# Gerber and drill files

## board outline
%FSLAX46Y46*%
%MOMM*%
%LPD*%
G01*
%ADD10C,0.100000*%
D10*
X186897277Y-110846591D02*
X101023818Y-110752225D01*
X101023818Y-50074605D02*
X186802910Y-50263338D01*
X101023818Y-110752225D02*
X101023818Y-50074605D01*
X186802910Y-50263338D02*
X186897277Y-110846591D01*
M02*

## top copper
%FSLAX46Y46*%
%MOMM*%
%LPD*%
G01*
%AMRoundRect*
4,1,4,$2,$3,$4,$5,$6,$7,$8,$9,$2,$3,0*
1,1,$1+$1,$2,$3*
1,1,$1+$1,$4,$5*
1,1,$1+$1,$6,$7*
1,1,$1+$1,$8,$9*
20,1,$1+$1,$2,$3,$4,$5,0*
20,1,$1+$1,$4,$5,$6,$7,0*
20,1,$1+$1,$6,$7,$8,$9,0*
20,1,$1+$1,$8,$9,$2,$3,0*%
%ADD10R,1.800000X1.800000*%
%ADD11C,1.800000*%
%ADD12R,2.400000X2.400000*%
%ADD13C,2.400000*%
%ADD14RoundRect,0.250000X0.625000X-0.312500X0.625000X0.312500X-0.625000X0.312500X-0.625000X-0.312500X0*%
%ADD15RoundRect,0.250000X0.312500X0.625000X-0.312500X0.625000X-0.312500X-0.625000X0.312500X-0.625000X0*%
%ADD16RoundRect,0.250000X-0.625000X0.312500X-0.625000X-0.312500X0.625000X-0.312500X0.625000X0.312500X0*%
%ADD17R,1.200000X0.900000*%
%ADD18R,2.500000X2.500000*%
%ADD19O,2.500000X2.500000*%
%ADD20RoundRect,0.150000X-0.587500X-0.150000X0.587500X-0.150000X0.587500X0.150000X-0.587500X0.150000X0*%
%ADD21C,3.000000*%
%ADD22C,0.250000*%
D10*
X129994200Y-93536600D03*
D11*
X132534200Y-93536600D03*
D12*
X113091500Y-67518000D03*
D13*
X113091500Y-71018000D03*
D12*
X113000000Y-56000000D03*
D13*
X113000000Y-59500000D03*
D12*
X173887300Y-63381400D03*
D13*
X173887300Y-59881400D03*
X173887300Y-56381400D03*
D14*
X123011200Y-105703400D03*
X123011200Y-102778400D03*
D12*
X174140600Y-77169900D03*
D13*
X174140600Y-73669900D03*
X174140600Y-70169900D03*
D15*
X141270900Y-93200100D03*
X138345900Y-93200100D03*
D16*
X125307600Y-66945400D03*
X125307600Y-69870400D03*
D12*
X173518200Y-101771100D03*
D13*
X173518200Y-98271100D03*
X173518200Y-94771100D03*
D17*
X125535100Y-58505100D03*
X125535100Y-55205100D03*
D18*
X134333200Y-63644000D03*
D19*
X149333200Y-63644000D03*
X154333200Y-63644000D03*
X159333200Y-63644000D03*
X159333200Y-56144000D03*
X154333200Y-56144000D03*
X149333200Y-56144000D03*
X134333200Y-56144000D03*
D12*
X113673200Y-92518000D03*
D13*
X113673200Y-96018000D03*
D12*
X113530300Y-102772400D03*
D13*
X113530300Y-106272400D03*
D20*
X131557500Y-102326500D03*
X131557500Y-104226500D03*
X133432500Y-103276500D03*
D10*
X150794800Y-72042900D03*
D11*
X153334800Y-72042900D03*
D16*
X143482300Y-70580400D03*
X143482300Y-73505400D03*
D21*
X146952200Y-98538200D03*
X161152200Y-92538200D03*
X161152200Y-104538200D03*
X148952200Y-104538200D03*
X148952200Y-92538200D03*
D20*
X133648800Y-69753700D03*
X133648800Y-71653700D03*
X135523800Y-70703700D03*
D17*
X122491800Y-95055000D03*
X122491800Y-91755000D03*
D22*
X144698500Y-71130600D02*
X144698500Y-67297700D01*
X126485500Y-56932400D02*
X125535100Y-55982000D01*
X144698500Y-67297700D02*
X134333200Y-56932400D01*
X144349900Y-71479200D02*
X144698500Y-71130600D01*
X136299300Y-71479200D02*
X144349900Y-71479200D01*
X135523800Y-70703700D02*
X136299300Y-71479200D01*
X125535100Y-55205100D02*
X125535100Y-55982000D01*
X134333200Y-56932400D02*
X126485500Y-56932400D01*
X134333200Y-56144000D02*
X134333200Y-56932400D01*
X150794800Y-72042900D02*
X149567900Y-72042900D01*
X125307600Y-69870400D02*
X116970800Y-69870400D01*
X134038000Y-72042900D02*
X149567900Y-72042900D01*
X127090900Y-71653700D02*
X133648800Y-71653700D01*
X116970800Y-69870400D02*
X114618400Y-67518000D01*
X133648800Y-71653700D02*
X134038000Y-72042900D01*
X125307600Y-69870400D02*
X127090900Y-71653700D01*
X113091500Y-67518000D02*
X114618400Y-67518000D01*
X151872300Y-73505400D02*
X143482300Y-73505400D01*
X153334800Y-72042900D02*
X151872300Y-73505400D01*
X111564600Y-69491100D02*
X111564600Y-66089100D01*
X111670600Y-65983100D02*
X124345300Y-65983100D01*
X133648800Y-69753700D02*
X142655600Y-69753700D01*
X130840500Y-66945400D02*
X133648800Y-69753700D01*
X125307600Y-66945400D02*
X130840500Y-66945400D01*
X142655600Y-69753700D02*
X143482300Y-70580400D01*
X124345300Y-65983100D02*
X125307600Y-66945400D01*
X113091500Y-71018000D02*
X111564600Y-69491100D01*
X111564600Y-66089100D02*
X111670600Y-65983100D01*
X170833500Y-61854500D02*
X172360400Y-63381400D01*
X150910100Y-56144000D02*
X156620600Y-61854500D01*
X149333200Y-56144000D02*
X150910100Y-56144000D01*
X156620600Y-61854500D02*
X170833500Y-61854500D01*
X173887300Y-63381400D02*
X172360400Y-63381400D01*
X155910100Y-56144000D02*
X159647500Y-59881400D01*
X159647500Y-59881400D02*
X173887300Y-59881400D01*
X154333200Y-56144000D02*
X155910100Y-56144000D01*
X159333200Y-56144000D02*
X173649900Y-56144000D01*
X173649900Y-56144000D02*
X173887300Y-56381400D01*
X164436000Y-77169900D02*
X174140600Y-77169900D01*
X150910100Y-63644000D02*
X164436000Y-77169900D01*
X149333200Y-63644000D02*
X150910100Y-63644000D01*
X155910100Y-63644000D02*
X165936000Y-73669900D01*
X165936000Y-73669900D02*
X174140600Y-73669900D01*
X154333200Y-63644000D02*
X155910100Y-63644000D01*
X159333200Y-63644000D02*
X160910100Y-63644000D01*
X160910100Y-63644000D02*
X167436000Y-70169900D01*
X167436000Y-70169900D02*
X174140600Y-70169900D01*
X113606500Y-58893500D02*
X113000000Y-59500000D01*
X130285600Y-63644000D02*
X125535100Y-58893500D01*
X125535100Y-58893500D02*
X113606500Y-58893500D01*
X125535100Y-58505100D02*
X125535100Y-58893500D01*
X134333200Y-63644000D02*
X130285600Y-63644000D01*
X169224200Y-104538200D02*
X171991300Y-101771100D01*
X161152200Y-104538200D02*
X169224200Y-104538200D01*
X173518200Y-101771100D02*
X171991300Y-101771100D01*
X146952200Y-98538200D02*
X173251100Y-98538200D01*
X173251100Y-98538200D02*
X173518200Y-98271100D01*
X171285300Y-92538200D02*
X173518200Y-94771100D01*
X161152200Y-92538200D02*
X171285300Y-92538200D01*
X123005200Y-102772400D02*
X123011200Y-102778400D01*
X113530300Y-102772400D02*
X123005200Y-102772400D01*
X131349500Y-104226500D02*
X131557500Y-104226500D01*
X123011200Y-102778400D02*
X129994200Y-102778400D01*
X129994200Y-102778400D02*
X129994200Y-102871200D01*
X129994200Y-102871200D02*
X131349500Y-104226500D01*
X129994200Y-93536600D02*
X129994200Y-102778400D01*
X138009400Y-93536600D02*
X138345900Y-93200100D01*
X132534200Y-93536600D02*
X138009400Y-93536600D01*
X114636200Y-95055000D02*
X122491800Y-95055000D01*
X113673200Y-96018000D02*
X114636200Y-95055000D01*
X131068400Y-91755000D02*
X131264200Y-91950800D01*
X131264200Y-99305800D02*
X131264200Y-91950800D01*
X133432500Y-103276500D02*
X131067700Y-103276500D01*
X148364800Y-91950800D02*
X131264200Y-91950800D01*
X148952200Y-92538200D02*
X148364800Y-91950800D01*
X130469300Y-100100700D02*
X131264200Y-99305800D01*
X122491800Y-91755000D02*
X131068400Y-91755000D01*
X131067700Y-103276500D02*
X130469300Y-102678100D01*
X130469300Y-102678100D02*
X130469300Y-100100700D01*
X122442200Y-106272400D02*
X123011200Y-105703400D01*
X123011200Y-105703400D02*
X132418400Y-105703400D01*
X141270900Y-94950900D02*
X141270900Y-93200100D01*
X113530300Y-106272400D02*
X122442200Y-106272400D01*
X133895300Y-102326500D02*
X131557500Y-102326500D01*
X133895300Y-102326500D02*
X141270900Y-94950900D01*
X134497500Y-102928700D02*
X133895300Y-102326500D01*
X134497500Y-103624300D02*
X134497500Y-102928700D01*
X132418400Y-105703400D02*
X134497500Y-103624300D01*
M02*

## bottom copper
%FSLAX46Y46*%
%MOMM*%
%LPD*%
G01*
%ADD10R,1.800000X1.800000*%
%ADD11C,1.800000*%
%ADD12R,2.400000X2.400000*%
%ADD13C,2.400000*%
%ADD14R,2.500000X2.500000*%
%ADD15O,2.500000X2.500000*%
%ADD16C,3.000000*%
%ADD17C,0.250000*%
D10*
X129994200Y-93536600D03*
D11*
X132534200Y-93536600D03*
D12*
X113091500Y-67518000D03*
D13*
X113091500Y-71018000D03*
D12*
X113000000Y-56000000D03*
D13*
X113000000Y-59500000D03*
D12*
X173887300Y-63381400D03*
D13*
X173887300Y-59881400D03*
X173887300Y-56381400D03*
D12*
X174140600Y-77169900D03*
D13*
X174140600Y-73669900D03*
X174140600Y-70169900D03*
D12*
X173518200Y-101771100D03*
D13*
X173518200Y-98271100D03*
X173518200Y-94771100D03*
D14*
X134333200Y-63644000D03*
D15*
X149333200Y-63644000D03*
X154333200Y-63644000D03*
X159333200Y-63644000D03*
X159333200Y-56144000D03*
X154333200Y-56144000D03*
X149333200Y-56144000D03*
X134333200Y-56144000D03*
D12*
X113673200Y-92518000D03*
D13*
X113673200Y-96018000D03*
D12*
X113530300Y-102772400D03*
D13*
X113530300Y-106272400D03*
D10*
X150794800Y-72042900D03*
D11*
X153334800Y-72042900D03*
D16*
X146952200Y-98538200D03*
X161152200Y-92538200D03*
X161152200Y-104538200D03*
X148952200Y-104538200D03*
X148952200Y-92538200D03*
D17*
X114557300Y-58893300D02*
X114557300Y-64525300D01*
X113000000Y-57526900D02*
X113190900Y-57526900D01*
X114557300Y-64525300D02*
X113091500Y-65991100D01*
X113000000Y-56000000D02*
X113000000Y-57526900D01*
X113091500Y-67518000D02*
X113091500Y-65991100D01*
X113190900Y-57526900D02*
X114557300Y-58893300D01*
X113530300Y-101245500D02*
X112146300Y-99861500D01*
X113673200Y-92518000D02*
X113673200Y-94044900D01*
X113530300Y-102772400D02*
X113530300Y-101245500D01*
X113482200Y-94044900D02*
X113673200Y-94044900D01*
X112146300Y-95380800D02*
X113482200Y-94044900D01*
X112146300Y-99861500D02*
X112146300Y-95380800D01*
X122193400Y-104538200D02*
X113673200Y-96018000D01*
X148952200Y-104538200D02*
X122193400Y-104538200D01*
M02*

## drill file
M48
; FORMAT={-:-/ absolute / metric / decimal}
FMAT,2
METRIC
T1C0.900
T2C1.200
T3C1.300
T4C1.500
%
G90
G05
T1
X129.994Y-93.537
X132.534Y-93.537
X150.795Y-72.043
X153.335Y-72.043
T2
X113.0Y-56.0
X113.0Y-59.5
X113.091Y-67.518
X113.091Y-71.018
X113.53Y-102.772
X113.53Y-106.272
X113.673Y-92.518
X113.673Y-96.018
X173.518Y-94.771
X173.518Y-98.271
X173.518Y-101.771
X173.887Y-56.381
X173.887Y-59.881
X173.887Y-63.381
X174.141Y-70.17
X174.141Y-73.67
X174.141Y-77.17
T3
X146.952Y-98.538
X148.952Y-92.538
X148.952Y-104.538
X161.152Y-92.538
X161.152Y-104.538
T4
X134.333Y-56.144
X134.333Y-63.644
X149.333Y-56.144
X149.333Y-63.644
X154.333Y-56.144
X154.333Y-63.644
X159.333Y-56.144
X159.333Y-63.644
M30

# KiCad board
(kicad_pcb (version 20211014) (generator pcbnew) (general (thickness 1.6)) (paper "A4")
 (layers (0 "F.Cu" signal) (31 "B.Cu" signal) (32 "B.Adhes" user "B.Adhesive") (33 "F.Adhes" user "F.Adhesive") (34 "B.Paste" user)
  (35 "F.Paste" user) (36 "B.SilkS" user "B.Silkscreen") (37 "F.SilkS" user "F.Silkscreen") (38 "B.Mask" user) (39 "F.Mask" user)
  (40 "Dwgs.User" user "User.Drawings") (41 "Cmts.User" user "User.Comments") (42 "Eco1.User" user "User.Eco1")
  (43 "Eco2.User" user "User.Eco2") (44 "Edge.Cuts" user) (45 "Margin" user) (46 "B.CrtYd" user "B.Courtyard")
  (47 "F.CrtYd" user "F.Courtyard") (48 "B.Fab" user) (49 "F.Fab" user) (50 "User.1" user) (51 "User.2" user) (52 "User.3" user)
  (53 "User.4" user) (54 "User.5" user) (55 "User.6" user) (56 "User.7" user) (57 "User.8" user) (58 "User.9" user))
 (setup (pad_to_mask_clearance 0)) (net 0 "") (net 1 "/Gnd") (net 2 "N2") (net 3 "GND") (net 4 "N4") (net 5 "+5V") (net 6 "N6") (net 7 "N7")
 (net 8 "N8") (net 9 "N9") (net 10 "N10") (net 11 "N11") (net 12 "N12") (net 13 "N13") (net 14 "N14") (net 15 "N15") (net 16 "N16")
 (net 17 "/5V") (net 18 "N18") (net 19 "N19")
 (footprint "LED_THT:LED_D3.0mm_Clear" (layer "F.Cu") (at 129.9942 93.5366)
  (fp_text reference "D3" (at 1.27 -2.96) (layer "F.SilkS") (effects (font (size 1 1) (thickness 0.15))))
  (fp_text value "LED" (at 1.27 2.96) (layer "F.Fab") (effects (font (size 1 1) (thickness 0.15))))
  (pad "1" thru_hole rect (at 0 0) (size 1.8 1.8) (drill 0.9) (layers *.Cu *.Mask) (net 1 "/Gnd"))
  (pad "2" thru_hole circle (at 2.54 0) (size 1.8 1.8) (drill 0.9) (layers *.Cu *.Mask) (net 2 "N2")))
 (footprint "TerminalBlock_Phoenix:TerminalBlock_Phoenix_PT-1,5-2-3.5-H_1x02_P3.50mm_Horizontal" (layer "F.Cu") (at 113.0915 67.518 -90)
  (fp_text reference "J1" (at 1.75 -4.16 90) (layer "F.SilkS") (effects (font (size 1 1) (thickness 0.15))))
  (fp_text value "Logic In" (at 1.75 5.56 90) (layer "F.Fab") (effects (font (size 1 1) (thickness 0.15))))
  (pad "1" thru_hole rect (at 0 0 270) (size 2.4 2.4) (drill 1.2) (layers *.Cu *.Mask) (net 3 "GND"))
  (pad "2" thru_hole circle (at 3.5 0 270) (size 2.4 2.4) (drill 1.2) (layers *.Cu *.Mask) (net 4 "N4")))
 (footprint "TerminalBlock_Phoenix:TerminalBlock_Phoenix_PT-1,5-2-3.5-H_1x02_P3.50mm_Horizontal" (layer "F.Cu") (at 113 56 -90)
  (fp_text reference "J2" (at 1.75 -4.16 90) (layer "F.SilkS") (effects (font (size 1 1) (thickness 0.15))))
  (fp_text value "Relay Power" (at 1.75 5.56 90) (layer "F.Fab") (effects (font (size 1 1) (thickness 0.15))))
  (pad "1" thru_hole rect (at 0 0 270) (size 2.4 2.4) (drill 1.2) (layers *.Cu *.Mask) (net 3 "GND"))
  (pad "2" thru_hole circle (at 3.5 0 270) (size 2.4 2.4) (drill 1.2) (layers *.Cu *.Mask) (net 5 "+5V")))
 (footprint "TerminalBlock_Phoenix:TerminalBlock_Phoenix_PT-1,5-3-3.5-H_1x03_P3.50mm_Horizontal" (layer "F.Cu") (at 173.8873 63.3814 90)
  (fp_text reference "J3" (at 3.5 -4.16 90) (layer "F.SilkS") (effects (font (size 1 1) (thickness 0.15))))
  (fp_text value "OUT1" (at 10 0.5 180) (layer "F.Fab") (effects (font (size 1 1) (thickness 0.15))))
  (pad "1" thru_hole rect (at 0 0 90) (size 2.4 2.4) (drill 1.2) (layers *.Cu *.Mask) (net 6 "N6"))
  (pad "2" thru_hole circle (at 3.5 0 90) (size 2.4 2.4) (drill 1.2) (layers *.Cu *.Mask) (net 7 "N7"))
  (pad "3" thru_hole circle (at 7 0 90) (size 2.4 2.4) (drill 1.2) (layers *.Cu *.Mask) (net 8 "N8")))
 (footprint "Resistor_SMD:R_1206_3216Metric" (layer "F.Cu") (at 123.0112 104.2409 90)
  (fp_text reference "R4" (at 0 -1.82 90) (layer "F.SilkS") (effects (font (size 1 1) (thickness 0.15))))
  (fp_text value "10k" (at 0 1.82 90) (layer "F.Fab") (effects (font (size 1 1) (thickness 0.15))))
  (pad "1" smd roundrect (at -1.4625 0 90) (size 1.125 1.75) (layers "F.Cu" "F.Paste" "F.Mask") (roundrect_rratio 0.222222) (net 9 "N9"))
  (pad "2" smd roundrect (at 1.4625 0 90) (size 1.125 1.75) (layers "F.Cu" "F.Paste" "F.Mask") (roundrect_rratio 0.222222) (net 1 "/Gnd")))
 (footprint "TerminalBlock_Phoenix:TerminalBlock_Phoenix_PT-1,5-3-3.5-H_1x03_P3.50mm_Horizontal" (layer "F.Cu") (at 174.1406 77.1699 90)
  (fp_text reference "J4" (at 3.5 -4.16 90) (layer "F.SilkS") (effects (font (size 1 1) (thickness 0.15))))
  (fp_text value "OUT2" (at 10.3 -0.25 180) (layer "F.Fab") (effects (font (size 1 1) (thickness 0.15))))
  (pad "1" thru_hole rect (at 0 0 90) (size 2.4 2.4) (drill 1.2) (layers *.Cu *.Mask) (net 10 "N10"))
  (pad "2" thru_hole circle (at 3.5 0 90) (size 2.4 2.4) (drill 1.2) (layers *.Cu *.Mask) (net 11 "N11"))
  (pad "3" thru_hole circle (at 7 0 90) (size 2.4 2.4) (drill 1.2) (layers *.Cu *.Mask) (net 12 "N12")))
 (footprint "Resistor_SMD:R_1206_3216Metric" (layer "F.Cu") (at 139.8084 93.2001 180)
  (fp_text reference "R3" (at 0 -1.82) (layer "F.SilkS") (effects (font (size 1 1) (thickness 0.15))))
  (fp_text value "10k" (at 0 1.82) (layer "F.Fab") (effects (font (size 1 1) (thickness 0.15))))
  (pad "1" smd roundrect (at -1.4625 0 180) (size 1.125 1.75) (layers "F.Cu" "F.Paste" "F.Mask") (roundrect_rratio 0.222222) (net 9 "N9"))
  (pad "2" smd roundrect (at 1.4625 0 180) (size 1.125 1.75) (layers "F.Cu" "F.Paste" "F.Mask") (roundrect_rratio 0.222222) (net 2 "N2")))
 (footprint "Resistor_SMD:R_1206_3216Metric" (layer "F.Cu") (at 125.3076 68.4079 -90)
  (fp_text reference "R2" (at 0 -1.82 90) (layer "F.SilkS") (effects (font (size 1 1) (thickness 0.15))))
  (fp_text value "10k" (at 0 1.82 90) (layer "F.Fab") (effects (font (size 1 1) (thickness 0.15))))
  (pad "1" smd roundrect (at -1.4625 0 270) (size 1.125 1.75) (layers "F.Cu" "F.Paste" "F.Mask") (roundrect_rratio 0.2222222222)
   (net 4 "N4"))
  (pad "2" smd roundrect (at 1.4625 0 270) (size 1.125 1.75) (layers "F.Cu" "F.Paste" "F.Mask") (roundrect_rratio 0.2222222222)
   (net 3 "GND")))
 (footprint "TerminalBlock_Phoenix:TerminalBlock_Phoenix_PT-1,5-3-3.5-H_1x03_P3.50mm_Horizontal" (layer "F.Cu") (at 173.5182 101.7711 90)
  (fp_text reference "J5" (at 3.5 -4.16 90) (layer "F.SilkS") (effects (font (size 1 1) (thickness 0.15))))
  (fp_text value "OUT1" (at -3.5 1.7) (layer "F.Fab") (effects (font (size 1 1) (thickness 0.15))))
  (pad "1" thru_hole rect (at 0 0 90) (size 2.4 2.4) (drill 1.2) (layers *.Cu *.Mask) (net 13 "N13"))
  (pad "2" thru_hole circle (at 3.5 0 90) (size 2.4 2.4) (drill 1.2) (layers *.Cu *.Mask) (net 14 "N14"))
  (pad "3" thru_hole circle (at 7 0 90) (size 2.4 2.4) (drill 1.2) (layers *.Cu *.Mask) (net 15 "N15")))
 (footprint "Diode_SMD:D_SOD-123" (layer "F.Cu") (at 125.5351 56.8551 90)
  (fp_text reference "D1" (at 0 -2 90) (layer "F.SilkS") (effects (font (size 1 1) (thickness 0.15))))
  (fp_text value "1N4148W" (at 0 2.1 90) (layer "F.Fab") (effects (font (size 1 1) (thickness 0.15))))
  (pad "1" smd rect (at -1.65 0 90) (size 0.9 1.2) (layers "F.Cu" "F.Paste" "F.Mask") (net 5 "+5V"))
  (pad "2" smd rect (at 1.65 0 90) (size 0.9 1.2) (layers "F.Cu" "F.Paste" "F.Mask") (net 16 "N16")))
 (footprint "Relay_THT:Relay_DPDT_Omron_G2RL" (layer "F.Cu") (at 134.3332 63.644)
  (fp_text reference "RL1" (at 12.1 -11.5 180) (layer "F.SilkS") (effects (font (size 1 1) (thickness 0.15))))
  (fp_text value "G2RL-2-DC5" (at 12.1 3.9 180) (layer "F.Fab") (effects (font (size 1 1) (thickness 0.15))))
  (pad "1" thru_hole rect (at 0 0 90) (size 2.5 2.5) (drill 1.5) (layers *.Cu *.Mask) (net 5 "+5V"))
  (pad "2" thru_hole oval (at 15 0 90) (size 2.5 2.5) (drill 1.5) (layers *.Cu *.Mask) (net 10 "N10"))
  (pad "3" thru_hole oval (at 20 0 90) (size 2.5 2.5) (drill 1.5) (layers *.Cu *.Mask) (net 11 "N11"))
  (pad "4" thru_hole oval (at 25 0 90) (size 2.5 2.5) (drill 1.5) (layers *.Cu *.Mask) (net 12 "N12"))
  (pad "5" thru_hole oval (at 25 -7.5 90) (size 2.5 2.5) (drill 1.5) (layers *.Cu *.Mask) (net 8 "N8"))
  (pad "6" thru_hole oval (at 20 -7.5 90) (size 2.5 2.5) (drill 1.5) (layers *.Cu *.Mask) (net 7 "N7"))
  (pad "7" thru_hole oval (at 15 -7.5 90) (size 2.5 2.5) (drill 1.5) (layers *.Cu *.Mask) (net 6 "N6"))
  (pad "8" thru_hole oval (at 0 -7.5 90) (size 2.5 2.5) (drill 1.5) (layers *.Cu *.Mask) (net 16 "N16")))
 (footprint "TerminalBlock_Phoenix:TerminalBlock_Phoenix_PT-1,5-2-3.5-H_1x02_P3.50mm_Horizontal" (layer "F.Cu") (at 113.6732 92.518 -90)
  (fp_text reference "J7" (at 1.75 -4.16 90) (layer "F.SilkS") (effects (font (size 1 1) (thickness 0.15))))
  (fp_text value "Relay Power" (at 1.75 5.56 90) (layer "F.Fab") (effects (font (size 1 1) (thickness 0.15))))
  (pad "1" thru_hole rect (at 0 0 270) (size 2.4 2.4) (drill 1.2) (layers *.Cu *.Mask) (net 1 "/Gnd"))
  (pad "2" thru_hole circle (at 3.5 0 270) (size 2.4 2.4) (drill 1.2) (layers *.Cu *.Mask) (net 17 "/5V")))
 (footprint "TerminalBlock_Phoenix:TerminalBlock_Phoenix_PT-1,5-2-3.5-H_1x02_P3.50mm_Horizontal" (layer "F.Cu") (at 113.5303 102.7724 -90)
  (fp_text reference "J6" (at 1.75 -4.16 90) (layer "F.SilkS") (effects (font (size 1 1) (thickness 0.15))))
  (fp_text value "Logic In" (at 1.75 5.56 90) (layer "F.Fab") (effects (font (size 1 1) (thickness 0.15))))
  (pad "1" thru_hole rect (at 0 0 270) (size 2.4 2.4) (drill 1.2) (layers *.Cu *.Mask) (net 1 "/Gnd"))
  (pad "2" thru_hole circle (at 3.5 0 270) (size 2.4 2.4) (drill 1.2) (layers *.Cu *.Mask) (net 9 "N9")))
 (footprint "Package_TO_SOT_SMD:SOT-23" (layer "F.Cu") (at 132.495 103.2765)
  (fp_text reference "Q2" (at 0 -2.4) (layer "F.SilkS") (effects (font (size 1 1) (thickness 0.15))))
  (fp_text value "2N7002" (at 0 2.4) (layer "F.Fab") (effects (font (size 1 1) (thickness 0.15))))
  (pad "1" smd roundrect (at -0.9375 -0.95) (size 1.475 0.6) (layers "F.Cu" "F.Paste" "F.Mask") (roundrect_rratio 0.25) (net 9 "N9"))
  (pad "2" smd roundrect (at -0.9375 0.95) (size 1.475 0.6) (layers "F.Cu" "F.Paste" "F.Mask") (roundrect_rratio 0.25) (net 1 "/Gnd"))
  (pad "3" smd roundrect (at 0.9375 0) (size 1.475 0.6) (layers "F.Cu" "F.Paste" "F.Mask") (roundrect_rratio 0.25) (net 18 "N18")))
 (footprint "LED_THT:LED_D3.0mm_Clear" (layer "F.Cu") (at 150.7948 72.0429)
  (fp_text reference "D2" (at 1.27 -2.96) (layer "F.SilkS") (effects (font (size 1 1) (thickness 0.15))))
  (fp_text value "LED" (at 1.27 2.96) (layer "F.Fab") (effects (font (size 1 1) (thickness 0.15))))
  (pad "1" thru_hole rect (at 0 0) (size 1.8 1.8) (drill 0.9) (layers *.Cu *.Mask) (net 3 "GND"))
  (pad "2" thru_hole circle (at 2.54 0) (size 1.8 1.8) (drill 0.9) (layers *.Cu *.Mask) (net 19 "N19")))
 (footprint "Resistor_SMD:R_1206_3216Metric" (layer "F.Cu") (at 143.4823 72.0429 -90)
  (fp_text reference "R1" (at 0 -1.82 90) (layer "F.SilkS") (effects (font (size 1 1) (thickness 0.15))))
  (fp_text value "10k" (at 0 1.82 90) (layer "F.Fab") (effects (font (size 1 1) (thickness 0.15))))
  (pad "1" smd roundrect (at -1.4625 0 270) (size 1.125 1.75) (layers "F.Cu" "F.Paste" "F.Mask") (roundrect_rratio 0.2222222222)
   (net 4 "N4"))
  (pad "2" smd roundrect (at 1.4625 0 270) (size 1.125 1.75) (layers "F.Cu" "F.Paste" "F.Mask") (roundrect_rratio 0.2222222222)
   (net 19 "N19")))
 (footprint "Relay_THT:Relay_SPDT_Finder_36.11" (layer "F.Cu") (at 146.9522 98.5382)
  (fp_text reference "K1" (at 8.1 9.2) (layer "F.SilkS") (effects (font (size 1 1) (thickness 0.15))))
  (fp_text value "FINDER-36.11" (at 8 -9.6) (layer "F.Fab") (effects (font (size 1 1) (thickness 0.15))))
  (pad "11" thru_hole circle (at 0 0) (size 3 3) (drill 1.3) (layers *.Cu *.Mask) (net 14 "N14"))
  (pad "12" thru_hole circle (at 14.2 -6) (size 3 3) (drill 1.3) (layers *.Cu *.Mask) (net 15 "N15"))
  (pad "14" thru_hole circle (at 14.2 6) (size 3 3) (drill 1.3) (layers *.Cu *.Mask) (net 13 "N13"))
  (pad "A1" thru_hole circle (at 2 6) (size 3 3) (drill 1.3) (layers *.Cu *.Mask) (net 17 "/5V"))
  (pad "A2" thru_hole circle (at 2 -6) (size 3 3) (drill 1.3) (layers *.Cu *.Mask) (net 18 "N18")))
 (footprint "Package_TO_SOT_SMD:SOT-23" (layer "F.Cu") (at 134.5863 70.7037)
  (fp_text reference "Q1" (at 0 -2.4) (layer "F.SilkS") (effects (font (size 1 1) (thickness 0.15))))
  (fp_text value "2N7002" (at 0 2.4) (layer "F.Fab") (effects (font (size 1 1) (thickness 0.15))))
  (pad "1" smd roundrect (at -0.9375 -0.95) (size 1.475 0.6) (layers "F.Cu" "F.Paste" "F.Mask") (roundrect_rratio 0.25) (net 4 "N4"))
  (pad "2" smd roundrect (at -0.9375 0.95) (size 1.475 0.6) (layers "F.Cu" "F.Paste" "F.Mask") (roundrect_rratio 0.25) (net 3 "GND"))
  (pad "3" smd roundrect (at 0.9375 0) (size 1.475 0.6) (layers "F.Cu" "F.Paste" "F.Mask") (roundrect_rratio 0.25) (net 16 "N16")))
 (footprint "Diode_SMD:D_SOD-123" (layer "F.Cu") (at 122.4918 93.405 90)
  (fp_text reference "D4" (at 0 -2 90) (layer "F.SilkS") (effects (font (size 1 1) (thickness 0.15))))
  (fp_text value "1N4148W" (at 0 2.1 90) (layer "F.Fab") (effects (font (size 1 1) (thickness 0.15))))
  (pad "1" smd rect (at -1.65 0 90) (size 0.9 1.2) (layers "F.Cu" "F.Paste" "F.Mask") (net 17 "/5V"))
  (pad "2" smd rect (at 1.65 0 90) (size 0.9 1.2) (layers "F.Cu" "F.Paste" "F.Mask") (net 18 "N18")))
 (gr_line (start 186.897277 110.846591) (end 101.023818 110.752225) (layer "Edge.Cuts") (width 0.1))
 (gr_line (start 101.023818 50.074605) (end 186.80291 50.263338) (layer "Edge.Cuts") (width 0.1))
 (gr_line (start 101.023818 110.752225) (end 101.023818 50.074605) (layer "Edge.Cuts") (width 0.1))
 (gr_line (start 186.80291 50.263338) (end 186.897277 110.846591) (layer "Edge.Cuts") (width 0.1))
 (segment (start 144.6985 71.1306) (end 144.6985 67.2977) (width 0.25) (layer "F.Cu") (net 16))
 (segment (start 126.4855 56.9324) (end 125.5351 55.982) (width 0.25) (layer "F.Cu") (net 16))
 (segment (start 144.6985 67.2977) (end 134.3332 56.9324) (width 0.25) (layer "F.Cu") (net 16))
 (segment (start 144.3499 71.4792) (end 144.6985 71.1306) (width 0.25) (layer "F.Cu") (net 16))
 (segment (start 136.2993 71.4792) (end 144.3499 71.4792) (width 0.25) (layer "F.Cu") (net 16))
 (segment (start 135.5238 70.7037) (end 136.2993 71.4792) (width 0.25) (layer "F.Cu") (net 16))
 (segment (start 125.5351 55.2051) (end 125.5351 55.982) (width 0.25) (layer "F.Cu") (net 16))
 (segment (start 134.3332 56.9324) (end 126.4855 56.9324) (width 0.25) (layer "F.Cu") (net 16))
 (segment (start 134.3332 56.144) (end 134.3332 56.9324) (width 0.25) (layer "F.Cu") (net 16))
 (segment (start 150.7948 72.0429) (end 149.5679 72.0429) (width 0.25) (layer "F.Cu") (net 3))
 (segment (start 125.3076 69.8704) (end 116.9708 69.8704) (width 0.25) (layer "F.Cu") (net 3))
 (segment (start 134.038 72.0429) (end 149.5679 72.0429) (width 0.25) (layer "F.Cu") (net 3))
 (segment (start 127.0909 71.6537) (end 133.6488 71.6537) (width 0.25) (layer "F.Cu") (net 3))
 (segment (start 116.9708 69.8704) (end 114.6184 67.518) (width 0.25) (layer "F.Cu") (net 3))
 (segment (start 133.6488 71.6537) (end 134.038 72.0429) (width 0.25) (layer "F.Cu") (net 3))
 (segment (start 125.3076 69.8704) (end 127.0909 71.6537) (width 0.25) (layer "F.Cu") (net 3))
 (segment (start 113.0915 67.518) (end 114.6184 67.518) (width 0.25) (layer "F.Cu") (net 3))
 (segment (start 114.5573 58.8933) (end 114.5573 64.5253) (width 0.25) (layer "B.Cu") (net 3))
 (segment (start 113 57.5269) (end 113.1909 57.5269) (width 0.25) (layer "B.Cu") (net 3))
 (segment (start 114.5573 64.5253) (end 113.0915 65.9911) (width 0.25) (layer "B.Cu") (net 3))
 (segment (start 113 56) (end 113 57.5269) (width 0.25) (layer "B.Cu") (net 3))
 (segment (start 113.0915 67.518) (end 113.0915 65.9911) (width 0.25) (layer "B.Cu") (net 3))
 (segment (start 113.1909 57.5269) (end 114.5573 58.8933) (width 0.25) (layer "B.Cu") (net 3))
 (segment (start 151.8723 73.5054) (end 143.4823 73.5054) (width 0.25) (layer "F.Cu") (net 19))
 (segment (start 153.3348 72.0429) (end 151.8723 73.5054) (width 0.25) (layer "F.Cu") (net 19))
 (segment (start 111.5646 69.4911) (end 111.5646 66.0891) (width 0.25) (layer "F.Cu") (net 4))
 (segment (start 111.6706 65.9831) (end 124.3453 65.9831) (width 0.25) (layer "F.Cu") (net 4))
 (segment (start 133.6488 69.7537) (end 142.6556 69.7537) (width 0.25) (layer "F.Cu") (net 4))
 (segment (start 130.8405 66.9454) (end 133.6488 69.7537) (width 0.25) (layer "F.Cu") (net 4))
 (segment (start 125.3076 66.9454) (end 130.8405 66.9454) (width 0.25) (layer "F.Cu") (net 4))
 (segment (start 142.6556 69.7537) (end 143.4823 70.5804) (width 0.25) (layer "F.Cu") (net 4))
 (segment (start 124.3453 65.9831) (end 125.3076 66.9454) (width 0.25) (layer "F.Cu") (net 4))
 (segment (start 113.0915 71.018) (end 111.5646 69.4911) (width 0.25) (layer "F.Cu") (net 4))
 (segment (start 111.5646 66.0891) (end 111.6706 65.9831) (width 0.25) (layer "F.Cu") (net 4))
 (segment (start 170.8335 61.8545) (end 172.3604 63.3814) (width 0.25) (layer "F.Cu") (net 6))
 (segment (start 150.9101 56.144) (end 156.6206 61.8545) (width 0.25) (layer "F.Cu") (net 6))
 (segment (start 149.3332 56.144) (end 150.9101 56.144) (width 0.25) (layer "F.Cu") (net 6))
 (segment (start 156.6206 61.8545) (end 170.8335 61.8545) (width 0.25) (layer "F.Cu") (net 6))
 (segment (start 173.8873 63.3814) (end 172.3604 63.3814) (width 0.25) (layer "F.Cu") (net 6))
 (segment (start 155.9101 56.144) (end 159.6475 59.8814) (width 0.25) (layer "F.Cu") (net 7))
 (segment (start 159.6475 59.8814) (end 173.8873 59.8814) (width 0.25) (layer "F.Cu") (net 7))
 (segment (start 154.3332 56.144) (end 155.9101 56.144) (width 0.25) (layer "F.Cu") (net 7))
 (segment (start 159.3332 56.144) (end 173.6499 56.144) (width 0.25) (layer "F.Cu") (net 8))
 (segment (start 173.6499 56.144) (end 173.8873 56.3814) (width 0.25) (layer "F.Cu") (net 8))
 (segment (start 164.436 77.1699) (end 174.1406 77.1699) (width 0.25) (layer "F.Cu") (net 10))
 (segment (start 150.9101 63.644) (end 164.436 77.1699) (width 0.25) (layer "F.Cu") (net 10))
 (segment (start 149.3332 63.644) (end 150.9101 63.644) (width 0.25) (layer "F.Cu") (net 10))
 (segment (start 155.9101 63.644) (end 165.936 73.6699) (width 0.25) (layer "F.Cu") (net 11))
 (segment (start 165.936 73.6699) (end 174.1406 73.6699) (width 0.25) (layer "F.Cu") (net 11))
 (segment (start 154.3332 63.644) (end 155.9101 63.644) (width 0.25) (layer "F.Cu") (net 11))
 (segment (start 159.3332 63.644) (end 160.9101 63.644) (width 0.25) (layer "F.Cu") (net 12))
 (segment (start 160.9101 63.644) (end 167.436 70.1699) (width 0.25) (layer "F.Cu") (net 12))
 (segment (start 167.436 70.1699) (end 174.1406 70.1699) (width 0.25) (layer "F.Cu") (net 12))
 (segment (start 113.6065 58.8935) (end 113 59.5) (width 0.25) (layer "F.Cu") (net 5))
 (segment (start 130.2856 63.644) (end 125.5351 58.8935) (width 0.25) (layer "F.Cu") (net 5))
 (segment (start 125.5351 58.8935) (end 113.6065 58.8935) (width 0.25) (layer "F.Cu") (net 5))
 (segment (start 125.5351 58.5051) (end 125.5351 58.8935) (width 0.25) (layer "F.Cu") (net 5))
 (segment (start 134.3332 63.644) (end 130.2856 63.644) (width 0.25) (layer "F.Cu") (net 5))
 (segment (start 169.2242 104.5382) (end 171.9913 101.7711) (width 0.25) (layer "F.Cu") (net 13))
 (segment (start 161.1522 104.5382) (end 169.2242 104.5382) (width 0.25) (layer "F.Cu") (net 13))
 (segment (start 173.5182 101.7711) (end 171.9913 101.7711) (width 0.25) (layer "F.Cu") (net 13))
 (segment (start 146.9522 98.5382) (end 173.2511 98.5382) (width 0.25) (layer "F.Cu") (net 14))
 (segment (start 173.2511 98.5382) (end 173.5182 98.2711) (width 0.25) (layer "F.Cu") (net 14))
 (segment (start 171.2853 92.5382) (end 173.5182 94.7711) (width 0.25) (layer "F.Cu") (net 15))
 (segment (start 161.1522 92.5382) (end 171.2853 92.5382) (width 0.25) (layer "F.Cu") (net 15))
 (segment (start 123.0052 102.7724) (end 123.0112 102.7784) (width 0.25) (layer "F.Cu") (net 1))
 (segment (start 113.5303 102.7724) (end 123.0052 102.7724) (width 0.25) (layer "F.Cu") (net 1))
 (segment (start 131.3495 104.2265) (end 131.5575 104.2265) (width 0.25) (layer "F.Cu") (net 1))
 (segment (start 123.0112 102.7784) (end 129.9942 102.7784) (width 0.25) (layer "F.Cu") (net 1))
 (segment (start 129.9942 102.7784) (end 129.9942 102.8712) (width 0.25) (layer "F.Cu") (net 1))
 (segment (start 129.9942 102.8712) (end 131.3495 104.2265) (width 0.25) (layer "F.Cu") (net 1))
 (segment (start 129.9942 93.5366) (end 129.9942 102.7784) (width 0.25) (layer "F.Cu") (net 1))
 (segment (start 113.5303 101.2455) (end 112.1463 99.8615) (width 0.25) (layer "B.Cu") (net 1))
 (segment (start 113.6732 92.518) (end 113.6732 94.0449) (width 0.25) (layer "B.Cu") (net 1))
 (segment (start 113.5303 102.7724) (end 113.5303 101.2455) (width 0.25) (layer "B.Cu") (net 1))
 (segment (start 113.4822 94.0449) (end 113.6732 94.0449) (width 0.25) (layer "B.Cu") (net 1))
 (segment (start 112.1463 95.3808) (end 113.4822 94.0449) (width 0.25) (layer "B.Cu") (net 1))
 (segment (start 112.1463 99.8615) (end 112.1463 95.3808) (width 0.25) (layer "B.Cu") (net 1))
 (segment (start 138.0094 93.5366) (end 138.3459 93.2001) (width 0.25) (layer "F.Cu") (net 2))
 (segment (start 132.5342 93.5366) (end 138.0094 93.5366) (width 0.25) (layer "F.Cu") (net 2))
 (segment (start 114.6362 95.055) (end 122.4918 95.055) (width 0.25) (layer "F.Cu") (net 17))
 (segment (start 113.6732 96.018) (end 114.6362 95.055) (width 0.25) (layer "F.Cu") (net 17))
 (segment (start 122.1934 104.5382) (end 113.6732 96.018) (width 0.25) (layer "B.Cu") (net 17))
 (segment (start 148.9522 104.5382) (end 122.1934 104.5382) (width 0.25) (layer "B.Cu") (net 17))
 (segment (start 131.0684 91.755) (end 131.2642 91.9508) (width 0.25) (layer "F.Cu") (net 18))
 (segment (start 131.2642 99.3058) (end 131.2642 91.9508) (width 0.25) (layer "F.Cu") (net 18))
 (segment (start 133.4325 103.2765) (end 131.0677 103.2765) (width 0.25) (layer "F.Cu") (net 18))
 (segment (start 148.3648 91.9508) (end 131.2642 91.9508) (width 0.25) (layer "F.Cu") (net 18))
 (segment (start 148.9522 92.5382) (end 148.3648 91.9508) (width 0.25) (layer "F.Cu") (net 18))
 (segment (start 130.4693 100.1007) (end 131.2642 99.3058) (width 0.25) (layer "F.Cu") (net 18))
 (segment (start 122.4918 91.755) (end 131.0684 91.755) (width 0.25) (layer "F.Cu") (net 18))
 (segment (start 131.0677 103.2765) (end 130.4693 102.6781) (width 0.25) (layer "F.Cu") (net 18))
 (segment (start 130.4693 102.6781) (end 130.4693 100.1007) (width 0.25) (layer "F.Cu") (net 18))
 (segment (start 122.4422 106.2724) (end 123.0112 105.7034) (width 0.25) (layer "F.Cu") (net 9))
 (segment (start 123.0112 105.7034) (end 132.4184 105.7034) (width 0.25) (layer "F.Cu") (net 9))
 (segment (start 141.2709 94.9509) (end 141.2709 93.2001) (width 0.25) (layer "F.Cu") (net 9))
 (segment (start 113.5303 106.2724) (end 122.4422 106.2724) (width 0.25) (layer "F.Cu") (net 9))
 (segment (start 133.8953 102.3265) (end 131.5575 102.3265) (width 0.25) (layer "F.Cu") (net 9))
 (segment (start 133.8953 102.3265) (end 141.2709 94.9509) (width 0.25) (layer "F.Cu") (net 9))
 (segment (start 134.4975 102.9287) (end 133.8953 102.3265) (width 0.25) (layer "F.Cu") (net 9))
 (segment (start 134.4975 103.6243) (end 134.4975 102.9287) (width 0.25) (layer "F.Cu") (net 9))
 (segment (start 132.4184 105.7034) (end 134.4975 103.6243) (width 0.25) (layer "F.Cu") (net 9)))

